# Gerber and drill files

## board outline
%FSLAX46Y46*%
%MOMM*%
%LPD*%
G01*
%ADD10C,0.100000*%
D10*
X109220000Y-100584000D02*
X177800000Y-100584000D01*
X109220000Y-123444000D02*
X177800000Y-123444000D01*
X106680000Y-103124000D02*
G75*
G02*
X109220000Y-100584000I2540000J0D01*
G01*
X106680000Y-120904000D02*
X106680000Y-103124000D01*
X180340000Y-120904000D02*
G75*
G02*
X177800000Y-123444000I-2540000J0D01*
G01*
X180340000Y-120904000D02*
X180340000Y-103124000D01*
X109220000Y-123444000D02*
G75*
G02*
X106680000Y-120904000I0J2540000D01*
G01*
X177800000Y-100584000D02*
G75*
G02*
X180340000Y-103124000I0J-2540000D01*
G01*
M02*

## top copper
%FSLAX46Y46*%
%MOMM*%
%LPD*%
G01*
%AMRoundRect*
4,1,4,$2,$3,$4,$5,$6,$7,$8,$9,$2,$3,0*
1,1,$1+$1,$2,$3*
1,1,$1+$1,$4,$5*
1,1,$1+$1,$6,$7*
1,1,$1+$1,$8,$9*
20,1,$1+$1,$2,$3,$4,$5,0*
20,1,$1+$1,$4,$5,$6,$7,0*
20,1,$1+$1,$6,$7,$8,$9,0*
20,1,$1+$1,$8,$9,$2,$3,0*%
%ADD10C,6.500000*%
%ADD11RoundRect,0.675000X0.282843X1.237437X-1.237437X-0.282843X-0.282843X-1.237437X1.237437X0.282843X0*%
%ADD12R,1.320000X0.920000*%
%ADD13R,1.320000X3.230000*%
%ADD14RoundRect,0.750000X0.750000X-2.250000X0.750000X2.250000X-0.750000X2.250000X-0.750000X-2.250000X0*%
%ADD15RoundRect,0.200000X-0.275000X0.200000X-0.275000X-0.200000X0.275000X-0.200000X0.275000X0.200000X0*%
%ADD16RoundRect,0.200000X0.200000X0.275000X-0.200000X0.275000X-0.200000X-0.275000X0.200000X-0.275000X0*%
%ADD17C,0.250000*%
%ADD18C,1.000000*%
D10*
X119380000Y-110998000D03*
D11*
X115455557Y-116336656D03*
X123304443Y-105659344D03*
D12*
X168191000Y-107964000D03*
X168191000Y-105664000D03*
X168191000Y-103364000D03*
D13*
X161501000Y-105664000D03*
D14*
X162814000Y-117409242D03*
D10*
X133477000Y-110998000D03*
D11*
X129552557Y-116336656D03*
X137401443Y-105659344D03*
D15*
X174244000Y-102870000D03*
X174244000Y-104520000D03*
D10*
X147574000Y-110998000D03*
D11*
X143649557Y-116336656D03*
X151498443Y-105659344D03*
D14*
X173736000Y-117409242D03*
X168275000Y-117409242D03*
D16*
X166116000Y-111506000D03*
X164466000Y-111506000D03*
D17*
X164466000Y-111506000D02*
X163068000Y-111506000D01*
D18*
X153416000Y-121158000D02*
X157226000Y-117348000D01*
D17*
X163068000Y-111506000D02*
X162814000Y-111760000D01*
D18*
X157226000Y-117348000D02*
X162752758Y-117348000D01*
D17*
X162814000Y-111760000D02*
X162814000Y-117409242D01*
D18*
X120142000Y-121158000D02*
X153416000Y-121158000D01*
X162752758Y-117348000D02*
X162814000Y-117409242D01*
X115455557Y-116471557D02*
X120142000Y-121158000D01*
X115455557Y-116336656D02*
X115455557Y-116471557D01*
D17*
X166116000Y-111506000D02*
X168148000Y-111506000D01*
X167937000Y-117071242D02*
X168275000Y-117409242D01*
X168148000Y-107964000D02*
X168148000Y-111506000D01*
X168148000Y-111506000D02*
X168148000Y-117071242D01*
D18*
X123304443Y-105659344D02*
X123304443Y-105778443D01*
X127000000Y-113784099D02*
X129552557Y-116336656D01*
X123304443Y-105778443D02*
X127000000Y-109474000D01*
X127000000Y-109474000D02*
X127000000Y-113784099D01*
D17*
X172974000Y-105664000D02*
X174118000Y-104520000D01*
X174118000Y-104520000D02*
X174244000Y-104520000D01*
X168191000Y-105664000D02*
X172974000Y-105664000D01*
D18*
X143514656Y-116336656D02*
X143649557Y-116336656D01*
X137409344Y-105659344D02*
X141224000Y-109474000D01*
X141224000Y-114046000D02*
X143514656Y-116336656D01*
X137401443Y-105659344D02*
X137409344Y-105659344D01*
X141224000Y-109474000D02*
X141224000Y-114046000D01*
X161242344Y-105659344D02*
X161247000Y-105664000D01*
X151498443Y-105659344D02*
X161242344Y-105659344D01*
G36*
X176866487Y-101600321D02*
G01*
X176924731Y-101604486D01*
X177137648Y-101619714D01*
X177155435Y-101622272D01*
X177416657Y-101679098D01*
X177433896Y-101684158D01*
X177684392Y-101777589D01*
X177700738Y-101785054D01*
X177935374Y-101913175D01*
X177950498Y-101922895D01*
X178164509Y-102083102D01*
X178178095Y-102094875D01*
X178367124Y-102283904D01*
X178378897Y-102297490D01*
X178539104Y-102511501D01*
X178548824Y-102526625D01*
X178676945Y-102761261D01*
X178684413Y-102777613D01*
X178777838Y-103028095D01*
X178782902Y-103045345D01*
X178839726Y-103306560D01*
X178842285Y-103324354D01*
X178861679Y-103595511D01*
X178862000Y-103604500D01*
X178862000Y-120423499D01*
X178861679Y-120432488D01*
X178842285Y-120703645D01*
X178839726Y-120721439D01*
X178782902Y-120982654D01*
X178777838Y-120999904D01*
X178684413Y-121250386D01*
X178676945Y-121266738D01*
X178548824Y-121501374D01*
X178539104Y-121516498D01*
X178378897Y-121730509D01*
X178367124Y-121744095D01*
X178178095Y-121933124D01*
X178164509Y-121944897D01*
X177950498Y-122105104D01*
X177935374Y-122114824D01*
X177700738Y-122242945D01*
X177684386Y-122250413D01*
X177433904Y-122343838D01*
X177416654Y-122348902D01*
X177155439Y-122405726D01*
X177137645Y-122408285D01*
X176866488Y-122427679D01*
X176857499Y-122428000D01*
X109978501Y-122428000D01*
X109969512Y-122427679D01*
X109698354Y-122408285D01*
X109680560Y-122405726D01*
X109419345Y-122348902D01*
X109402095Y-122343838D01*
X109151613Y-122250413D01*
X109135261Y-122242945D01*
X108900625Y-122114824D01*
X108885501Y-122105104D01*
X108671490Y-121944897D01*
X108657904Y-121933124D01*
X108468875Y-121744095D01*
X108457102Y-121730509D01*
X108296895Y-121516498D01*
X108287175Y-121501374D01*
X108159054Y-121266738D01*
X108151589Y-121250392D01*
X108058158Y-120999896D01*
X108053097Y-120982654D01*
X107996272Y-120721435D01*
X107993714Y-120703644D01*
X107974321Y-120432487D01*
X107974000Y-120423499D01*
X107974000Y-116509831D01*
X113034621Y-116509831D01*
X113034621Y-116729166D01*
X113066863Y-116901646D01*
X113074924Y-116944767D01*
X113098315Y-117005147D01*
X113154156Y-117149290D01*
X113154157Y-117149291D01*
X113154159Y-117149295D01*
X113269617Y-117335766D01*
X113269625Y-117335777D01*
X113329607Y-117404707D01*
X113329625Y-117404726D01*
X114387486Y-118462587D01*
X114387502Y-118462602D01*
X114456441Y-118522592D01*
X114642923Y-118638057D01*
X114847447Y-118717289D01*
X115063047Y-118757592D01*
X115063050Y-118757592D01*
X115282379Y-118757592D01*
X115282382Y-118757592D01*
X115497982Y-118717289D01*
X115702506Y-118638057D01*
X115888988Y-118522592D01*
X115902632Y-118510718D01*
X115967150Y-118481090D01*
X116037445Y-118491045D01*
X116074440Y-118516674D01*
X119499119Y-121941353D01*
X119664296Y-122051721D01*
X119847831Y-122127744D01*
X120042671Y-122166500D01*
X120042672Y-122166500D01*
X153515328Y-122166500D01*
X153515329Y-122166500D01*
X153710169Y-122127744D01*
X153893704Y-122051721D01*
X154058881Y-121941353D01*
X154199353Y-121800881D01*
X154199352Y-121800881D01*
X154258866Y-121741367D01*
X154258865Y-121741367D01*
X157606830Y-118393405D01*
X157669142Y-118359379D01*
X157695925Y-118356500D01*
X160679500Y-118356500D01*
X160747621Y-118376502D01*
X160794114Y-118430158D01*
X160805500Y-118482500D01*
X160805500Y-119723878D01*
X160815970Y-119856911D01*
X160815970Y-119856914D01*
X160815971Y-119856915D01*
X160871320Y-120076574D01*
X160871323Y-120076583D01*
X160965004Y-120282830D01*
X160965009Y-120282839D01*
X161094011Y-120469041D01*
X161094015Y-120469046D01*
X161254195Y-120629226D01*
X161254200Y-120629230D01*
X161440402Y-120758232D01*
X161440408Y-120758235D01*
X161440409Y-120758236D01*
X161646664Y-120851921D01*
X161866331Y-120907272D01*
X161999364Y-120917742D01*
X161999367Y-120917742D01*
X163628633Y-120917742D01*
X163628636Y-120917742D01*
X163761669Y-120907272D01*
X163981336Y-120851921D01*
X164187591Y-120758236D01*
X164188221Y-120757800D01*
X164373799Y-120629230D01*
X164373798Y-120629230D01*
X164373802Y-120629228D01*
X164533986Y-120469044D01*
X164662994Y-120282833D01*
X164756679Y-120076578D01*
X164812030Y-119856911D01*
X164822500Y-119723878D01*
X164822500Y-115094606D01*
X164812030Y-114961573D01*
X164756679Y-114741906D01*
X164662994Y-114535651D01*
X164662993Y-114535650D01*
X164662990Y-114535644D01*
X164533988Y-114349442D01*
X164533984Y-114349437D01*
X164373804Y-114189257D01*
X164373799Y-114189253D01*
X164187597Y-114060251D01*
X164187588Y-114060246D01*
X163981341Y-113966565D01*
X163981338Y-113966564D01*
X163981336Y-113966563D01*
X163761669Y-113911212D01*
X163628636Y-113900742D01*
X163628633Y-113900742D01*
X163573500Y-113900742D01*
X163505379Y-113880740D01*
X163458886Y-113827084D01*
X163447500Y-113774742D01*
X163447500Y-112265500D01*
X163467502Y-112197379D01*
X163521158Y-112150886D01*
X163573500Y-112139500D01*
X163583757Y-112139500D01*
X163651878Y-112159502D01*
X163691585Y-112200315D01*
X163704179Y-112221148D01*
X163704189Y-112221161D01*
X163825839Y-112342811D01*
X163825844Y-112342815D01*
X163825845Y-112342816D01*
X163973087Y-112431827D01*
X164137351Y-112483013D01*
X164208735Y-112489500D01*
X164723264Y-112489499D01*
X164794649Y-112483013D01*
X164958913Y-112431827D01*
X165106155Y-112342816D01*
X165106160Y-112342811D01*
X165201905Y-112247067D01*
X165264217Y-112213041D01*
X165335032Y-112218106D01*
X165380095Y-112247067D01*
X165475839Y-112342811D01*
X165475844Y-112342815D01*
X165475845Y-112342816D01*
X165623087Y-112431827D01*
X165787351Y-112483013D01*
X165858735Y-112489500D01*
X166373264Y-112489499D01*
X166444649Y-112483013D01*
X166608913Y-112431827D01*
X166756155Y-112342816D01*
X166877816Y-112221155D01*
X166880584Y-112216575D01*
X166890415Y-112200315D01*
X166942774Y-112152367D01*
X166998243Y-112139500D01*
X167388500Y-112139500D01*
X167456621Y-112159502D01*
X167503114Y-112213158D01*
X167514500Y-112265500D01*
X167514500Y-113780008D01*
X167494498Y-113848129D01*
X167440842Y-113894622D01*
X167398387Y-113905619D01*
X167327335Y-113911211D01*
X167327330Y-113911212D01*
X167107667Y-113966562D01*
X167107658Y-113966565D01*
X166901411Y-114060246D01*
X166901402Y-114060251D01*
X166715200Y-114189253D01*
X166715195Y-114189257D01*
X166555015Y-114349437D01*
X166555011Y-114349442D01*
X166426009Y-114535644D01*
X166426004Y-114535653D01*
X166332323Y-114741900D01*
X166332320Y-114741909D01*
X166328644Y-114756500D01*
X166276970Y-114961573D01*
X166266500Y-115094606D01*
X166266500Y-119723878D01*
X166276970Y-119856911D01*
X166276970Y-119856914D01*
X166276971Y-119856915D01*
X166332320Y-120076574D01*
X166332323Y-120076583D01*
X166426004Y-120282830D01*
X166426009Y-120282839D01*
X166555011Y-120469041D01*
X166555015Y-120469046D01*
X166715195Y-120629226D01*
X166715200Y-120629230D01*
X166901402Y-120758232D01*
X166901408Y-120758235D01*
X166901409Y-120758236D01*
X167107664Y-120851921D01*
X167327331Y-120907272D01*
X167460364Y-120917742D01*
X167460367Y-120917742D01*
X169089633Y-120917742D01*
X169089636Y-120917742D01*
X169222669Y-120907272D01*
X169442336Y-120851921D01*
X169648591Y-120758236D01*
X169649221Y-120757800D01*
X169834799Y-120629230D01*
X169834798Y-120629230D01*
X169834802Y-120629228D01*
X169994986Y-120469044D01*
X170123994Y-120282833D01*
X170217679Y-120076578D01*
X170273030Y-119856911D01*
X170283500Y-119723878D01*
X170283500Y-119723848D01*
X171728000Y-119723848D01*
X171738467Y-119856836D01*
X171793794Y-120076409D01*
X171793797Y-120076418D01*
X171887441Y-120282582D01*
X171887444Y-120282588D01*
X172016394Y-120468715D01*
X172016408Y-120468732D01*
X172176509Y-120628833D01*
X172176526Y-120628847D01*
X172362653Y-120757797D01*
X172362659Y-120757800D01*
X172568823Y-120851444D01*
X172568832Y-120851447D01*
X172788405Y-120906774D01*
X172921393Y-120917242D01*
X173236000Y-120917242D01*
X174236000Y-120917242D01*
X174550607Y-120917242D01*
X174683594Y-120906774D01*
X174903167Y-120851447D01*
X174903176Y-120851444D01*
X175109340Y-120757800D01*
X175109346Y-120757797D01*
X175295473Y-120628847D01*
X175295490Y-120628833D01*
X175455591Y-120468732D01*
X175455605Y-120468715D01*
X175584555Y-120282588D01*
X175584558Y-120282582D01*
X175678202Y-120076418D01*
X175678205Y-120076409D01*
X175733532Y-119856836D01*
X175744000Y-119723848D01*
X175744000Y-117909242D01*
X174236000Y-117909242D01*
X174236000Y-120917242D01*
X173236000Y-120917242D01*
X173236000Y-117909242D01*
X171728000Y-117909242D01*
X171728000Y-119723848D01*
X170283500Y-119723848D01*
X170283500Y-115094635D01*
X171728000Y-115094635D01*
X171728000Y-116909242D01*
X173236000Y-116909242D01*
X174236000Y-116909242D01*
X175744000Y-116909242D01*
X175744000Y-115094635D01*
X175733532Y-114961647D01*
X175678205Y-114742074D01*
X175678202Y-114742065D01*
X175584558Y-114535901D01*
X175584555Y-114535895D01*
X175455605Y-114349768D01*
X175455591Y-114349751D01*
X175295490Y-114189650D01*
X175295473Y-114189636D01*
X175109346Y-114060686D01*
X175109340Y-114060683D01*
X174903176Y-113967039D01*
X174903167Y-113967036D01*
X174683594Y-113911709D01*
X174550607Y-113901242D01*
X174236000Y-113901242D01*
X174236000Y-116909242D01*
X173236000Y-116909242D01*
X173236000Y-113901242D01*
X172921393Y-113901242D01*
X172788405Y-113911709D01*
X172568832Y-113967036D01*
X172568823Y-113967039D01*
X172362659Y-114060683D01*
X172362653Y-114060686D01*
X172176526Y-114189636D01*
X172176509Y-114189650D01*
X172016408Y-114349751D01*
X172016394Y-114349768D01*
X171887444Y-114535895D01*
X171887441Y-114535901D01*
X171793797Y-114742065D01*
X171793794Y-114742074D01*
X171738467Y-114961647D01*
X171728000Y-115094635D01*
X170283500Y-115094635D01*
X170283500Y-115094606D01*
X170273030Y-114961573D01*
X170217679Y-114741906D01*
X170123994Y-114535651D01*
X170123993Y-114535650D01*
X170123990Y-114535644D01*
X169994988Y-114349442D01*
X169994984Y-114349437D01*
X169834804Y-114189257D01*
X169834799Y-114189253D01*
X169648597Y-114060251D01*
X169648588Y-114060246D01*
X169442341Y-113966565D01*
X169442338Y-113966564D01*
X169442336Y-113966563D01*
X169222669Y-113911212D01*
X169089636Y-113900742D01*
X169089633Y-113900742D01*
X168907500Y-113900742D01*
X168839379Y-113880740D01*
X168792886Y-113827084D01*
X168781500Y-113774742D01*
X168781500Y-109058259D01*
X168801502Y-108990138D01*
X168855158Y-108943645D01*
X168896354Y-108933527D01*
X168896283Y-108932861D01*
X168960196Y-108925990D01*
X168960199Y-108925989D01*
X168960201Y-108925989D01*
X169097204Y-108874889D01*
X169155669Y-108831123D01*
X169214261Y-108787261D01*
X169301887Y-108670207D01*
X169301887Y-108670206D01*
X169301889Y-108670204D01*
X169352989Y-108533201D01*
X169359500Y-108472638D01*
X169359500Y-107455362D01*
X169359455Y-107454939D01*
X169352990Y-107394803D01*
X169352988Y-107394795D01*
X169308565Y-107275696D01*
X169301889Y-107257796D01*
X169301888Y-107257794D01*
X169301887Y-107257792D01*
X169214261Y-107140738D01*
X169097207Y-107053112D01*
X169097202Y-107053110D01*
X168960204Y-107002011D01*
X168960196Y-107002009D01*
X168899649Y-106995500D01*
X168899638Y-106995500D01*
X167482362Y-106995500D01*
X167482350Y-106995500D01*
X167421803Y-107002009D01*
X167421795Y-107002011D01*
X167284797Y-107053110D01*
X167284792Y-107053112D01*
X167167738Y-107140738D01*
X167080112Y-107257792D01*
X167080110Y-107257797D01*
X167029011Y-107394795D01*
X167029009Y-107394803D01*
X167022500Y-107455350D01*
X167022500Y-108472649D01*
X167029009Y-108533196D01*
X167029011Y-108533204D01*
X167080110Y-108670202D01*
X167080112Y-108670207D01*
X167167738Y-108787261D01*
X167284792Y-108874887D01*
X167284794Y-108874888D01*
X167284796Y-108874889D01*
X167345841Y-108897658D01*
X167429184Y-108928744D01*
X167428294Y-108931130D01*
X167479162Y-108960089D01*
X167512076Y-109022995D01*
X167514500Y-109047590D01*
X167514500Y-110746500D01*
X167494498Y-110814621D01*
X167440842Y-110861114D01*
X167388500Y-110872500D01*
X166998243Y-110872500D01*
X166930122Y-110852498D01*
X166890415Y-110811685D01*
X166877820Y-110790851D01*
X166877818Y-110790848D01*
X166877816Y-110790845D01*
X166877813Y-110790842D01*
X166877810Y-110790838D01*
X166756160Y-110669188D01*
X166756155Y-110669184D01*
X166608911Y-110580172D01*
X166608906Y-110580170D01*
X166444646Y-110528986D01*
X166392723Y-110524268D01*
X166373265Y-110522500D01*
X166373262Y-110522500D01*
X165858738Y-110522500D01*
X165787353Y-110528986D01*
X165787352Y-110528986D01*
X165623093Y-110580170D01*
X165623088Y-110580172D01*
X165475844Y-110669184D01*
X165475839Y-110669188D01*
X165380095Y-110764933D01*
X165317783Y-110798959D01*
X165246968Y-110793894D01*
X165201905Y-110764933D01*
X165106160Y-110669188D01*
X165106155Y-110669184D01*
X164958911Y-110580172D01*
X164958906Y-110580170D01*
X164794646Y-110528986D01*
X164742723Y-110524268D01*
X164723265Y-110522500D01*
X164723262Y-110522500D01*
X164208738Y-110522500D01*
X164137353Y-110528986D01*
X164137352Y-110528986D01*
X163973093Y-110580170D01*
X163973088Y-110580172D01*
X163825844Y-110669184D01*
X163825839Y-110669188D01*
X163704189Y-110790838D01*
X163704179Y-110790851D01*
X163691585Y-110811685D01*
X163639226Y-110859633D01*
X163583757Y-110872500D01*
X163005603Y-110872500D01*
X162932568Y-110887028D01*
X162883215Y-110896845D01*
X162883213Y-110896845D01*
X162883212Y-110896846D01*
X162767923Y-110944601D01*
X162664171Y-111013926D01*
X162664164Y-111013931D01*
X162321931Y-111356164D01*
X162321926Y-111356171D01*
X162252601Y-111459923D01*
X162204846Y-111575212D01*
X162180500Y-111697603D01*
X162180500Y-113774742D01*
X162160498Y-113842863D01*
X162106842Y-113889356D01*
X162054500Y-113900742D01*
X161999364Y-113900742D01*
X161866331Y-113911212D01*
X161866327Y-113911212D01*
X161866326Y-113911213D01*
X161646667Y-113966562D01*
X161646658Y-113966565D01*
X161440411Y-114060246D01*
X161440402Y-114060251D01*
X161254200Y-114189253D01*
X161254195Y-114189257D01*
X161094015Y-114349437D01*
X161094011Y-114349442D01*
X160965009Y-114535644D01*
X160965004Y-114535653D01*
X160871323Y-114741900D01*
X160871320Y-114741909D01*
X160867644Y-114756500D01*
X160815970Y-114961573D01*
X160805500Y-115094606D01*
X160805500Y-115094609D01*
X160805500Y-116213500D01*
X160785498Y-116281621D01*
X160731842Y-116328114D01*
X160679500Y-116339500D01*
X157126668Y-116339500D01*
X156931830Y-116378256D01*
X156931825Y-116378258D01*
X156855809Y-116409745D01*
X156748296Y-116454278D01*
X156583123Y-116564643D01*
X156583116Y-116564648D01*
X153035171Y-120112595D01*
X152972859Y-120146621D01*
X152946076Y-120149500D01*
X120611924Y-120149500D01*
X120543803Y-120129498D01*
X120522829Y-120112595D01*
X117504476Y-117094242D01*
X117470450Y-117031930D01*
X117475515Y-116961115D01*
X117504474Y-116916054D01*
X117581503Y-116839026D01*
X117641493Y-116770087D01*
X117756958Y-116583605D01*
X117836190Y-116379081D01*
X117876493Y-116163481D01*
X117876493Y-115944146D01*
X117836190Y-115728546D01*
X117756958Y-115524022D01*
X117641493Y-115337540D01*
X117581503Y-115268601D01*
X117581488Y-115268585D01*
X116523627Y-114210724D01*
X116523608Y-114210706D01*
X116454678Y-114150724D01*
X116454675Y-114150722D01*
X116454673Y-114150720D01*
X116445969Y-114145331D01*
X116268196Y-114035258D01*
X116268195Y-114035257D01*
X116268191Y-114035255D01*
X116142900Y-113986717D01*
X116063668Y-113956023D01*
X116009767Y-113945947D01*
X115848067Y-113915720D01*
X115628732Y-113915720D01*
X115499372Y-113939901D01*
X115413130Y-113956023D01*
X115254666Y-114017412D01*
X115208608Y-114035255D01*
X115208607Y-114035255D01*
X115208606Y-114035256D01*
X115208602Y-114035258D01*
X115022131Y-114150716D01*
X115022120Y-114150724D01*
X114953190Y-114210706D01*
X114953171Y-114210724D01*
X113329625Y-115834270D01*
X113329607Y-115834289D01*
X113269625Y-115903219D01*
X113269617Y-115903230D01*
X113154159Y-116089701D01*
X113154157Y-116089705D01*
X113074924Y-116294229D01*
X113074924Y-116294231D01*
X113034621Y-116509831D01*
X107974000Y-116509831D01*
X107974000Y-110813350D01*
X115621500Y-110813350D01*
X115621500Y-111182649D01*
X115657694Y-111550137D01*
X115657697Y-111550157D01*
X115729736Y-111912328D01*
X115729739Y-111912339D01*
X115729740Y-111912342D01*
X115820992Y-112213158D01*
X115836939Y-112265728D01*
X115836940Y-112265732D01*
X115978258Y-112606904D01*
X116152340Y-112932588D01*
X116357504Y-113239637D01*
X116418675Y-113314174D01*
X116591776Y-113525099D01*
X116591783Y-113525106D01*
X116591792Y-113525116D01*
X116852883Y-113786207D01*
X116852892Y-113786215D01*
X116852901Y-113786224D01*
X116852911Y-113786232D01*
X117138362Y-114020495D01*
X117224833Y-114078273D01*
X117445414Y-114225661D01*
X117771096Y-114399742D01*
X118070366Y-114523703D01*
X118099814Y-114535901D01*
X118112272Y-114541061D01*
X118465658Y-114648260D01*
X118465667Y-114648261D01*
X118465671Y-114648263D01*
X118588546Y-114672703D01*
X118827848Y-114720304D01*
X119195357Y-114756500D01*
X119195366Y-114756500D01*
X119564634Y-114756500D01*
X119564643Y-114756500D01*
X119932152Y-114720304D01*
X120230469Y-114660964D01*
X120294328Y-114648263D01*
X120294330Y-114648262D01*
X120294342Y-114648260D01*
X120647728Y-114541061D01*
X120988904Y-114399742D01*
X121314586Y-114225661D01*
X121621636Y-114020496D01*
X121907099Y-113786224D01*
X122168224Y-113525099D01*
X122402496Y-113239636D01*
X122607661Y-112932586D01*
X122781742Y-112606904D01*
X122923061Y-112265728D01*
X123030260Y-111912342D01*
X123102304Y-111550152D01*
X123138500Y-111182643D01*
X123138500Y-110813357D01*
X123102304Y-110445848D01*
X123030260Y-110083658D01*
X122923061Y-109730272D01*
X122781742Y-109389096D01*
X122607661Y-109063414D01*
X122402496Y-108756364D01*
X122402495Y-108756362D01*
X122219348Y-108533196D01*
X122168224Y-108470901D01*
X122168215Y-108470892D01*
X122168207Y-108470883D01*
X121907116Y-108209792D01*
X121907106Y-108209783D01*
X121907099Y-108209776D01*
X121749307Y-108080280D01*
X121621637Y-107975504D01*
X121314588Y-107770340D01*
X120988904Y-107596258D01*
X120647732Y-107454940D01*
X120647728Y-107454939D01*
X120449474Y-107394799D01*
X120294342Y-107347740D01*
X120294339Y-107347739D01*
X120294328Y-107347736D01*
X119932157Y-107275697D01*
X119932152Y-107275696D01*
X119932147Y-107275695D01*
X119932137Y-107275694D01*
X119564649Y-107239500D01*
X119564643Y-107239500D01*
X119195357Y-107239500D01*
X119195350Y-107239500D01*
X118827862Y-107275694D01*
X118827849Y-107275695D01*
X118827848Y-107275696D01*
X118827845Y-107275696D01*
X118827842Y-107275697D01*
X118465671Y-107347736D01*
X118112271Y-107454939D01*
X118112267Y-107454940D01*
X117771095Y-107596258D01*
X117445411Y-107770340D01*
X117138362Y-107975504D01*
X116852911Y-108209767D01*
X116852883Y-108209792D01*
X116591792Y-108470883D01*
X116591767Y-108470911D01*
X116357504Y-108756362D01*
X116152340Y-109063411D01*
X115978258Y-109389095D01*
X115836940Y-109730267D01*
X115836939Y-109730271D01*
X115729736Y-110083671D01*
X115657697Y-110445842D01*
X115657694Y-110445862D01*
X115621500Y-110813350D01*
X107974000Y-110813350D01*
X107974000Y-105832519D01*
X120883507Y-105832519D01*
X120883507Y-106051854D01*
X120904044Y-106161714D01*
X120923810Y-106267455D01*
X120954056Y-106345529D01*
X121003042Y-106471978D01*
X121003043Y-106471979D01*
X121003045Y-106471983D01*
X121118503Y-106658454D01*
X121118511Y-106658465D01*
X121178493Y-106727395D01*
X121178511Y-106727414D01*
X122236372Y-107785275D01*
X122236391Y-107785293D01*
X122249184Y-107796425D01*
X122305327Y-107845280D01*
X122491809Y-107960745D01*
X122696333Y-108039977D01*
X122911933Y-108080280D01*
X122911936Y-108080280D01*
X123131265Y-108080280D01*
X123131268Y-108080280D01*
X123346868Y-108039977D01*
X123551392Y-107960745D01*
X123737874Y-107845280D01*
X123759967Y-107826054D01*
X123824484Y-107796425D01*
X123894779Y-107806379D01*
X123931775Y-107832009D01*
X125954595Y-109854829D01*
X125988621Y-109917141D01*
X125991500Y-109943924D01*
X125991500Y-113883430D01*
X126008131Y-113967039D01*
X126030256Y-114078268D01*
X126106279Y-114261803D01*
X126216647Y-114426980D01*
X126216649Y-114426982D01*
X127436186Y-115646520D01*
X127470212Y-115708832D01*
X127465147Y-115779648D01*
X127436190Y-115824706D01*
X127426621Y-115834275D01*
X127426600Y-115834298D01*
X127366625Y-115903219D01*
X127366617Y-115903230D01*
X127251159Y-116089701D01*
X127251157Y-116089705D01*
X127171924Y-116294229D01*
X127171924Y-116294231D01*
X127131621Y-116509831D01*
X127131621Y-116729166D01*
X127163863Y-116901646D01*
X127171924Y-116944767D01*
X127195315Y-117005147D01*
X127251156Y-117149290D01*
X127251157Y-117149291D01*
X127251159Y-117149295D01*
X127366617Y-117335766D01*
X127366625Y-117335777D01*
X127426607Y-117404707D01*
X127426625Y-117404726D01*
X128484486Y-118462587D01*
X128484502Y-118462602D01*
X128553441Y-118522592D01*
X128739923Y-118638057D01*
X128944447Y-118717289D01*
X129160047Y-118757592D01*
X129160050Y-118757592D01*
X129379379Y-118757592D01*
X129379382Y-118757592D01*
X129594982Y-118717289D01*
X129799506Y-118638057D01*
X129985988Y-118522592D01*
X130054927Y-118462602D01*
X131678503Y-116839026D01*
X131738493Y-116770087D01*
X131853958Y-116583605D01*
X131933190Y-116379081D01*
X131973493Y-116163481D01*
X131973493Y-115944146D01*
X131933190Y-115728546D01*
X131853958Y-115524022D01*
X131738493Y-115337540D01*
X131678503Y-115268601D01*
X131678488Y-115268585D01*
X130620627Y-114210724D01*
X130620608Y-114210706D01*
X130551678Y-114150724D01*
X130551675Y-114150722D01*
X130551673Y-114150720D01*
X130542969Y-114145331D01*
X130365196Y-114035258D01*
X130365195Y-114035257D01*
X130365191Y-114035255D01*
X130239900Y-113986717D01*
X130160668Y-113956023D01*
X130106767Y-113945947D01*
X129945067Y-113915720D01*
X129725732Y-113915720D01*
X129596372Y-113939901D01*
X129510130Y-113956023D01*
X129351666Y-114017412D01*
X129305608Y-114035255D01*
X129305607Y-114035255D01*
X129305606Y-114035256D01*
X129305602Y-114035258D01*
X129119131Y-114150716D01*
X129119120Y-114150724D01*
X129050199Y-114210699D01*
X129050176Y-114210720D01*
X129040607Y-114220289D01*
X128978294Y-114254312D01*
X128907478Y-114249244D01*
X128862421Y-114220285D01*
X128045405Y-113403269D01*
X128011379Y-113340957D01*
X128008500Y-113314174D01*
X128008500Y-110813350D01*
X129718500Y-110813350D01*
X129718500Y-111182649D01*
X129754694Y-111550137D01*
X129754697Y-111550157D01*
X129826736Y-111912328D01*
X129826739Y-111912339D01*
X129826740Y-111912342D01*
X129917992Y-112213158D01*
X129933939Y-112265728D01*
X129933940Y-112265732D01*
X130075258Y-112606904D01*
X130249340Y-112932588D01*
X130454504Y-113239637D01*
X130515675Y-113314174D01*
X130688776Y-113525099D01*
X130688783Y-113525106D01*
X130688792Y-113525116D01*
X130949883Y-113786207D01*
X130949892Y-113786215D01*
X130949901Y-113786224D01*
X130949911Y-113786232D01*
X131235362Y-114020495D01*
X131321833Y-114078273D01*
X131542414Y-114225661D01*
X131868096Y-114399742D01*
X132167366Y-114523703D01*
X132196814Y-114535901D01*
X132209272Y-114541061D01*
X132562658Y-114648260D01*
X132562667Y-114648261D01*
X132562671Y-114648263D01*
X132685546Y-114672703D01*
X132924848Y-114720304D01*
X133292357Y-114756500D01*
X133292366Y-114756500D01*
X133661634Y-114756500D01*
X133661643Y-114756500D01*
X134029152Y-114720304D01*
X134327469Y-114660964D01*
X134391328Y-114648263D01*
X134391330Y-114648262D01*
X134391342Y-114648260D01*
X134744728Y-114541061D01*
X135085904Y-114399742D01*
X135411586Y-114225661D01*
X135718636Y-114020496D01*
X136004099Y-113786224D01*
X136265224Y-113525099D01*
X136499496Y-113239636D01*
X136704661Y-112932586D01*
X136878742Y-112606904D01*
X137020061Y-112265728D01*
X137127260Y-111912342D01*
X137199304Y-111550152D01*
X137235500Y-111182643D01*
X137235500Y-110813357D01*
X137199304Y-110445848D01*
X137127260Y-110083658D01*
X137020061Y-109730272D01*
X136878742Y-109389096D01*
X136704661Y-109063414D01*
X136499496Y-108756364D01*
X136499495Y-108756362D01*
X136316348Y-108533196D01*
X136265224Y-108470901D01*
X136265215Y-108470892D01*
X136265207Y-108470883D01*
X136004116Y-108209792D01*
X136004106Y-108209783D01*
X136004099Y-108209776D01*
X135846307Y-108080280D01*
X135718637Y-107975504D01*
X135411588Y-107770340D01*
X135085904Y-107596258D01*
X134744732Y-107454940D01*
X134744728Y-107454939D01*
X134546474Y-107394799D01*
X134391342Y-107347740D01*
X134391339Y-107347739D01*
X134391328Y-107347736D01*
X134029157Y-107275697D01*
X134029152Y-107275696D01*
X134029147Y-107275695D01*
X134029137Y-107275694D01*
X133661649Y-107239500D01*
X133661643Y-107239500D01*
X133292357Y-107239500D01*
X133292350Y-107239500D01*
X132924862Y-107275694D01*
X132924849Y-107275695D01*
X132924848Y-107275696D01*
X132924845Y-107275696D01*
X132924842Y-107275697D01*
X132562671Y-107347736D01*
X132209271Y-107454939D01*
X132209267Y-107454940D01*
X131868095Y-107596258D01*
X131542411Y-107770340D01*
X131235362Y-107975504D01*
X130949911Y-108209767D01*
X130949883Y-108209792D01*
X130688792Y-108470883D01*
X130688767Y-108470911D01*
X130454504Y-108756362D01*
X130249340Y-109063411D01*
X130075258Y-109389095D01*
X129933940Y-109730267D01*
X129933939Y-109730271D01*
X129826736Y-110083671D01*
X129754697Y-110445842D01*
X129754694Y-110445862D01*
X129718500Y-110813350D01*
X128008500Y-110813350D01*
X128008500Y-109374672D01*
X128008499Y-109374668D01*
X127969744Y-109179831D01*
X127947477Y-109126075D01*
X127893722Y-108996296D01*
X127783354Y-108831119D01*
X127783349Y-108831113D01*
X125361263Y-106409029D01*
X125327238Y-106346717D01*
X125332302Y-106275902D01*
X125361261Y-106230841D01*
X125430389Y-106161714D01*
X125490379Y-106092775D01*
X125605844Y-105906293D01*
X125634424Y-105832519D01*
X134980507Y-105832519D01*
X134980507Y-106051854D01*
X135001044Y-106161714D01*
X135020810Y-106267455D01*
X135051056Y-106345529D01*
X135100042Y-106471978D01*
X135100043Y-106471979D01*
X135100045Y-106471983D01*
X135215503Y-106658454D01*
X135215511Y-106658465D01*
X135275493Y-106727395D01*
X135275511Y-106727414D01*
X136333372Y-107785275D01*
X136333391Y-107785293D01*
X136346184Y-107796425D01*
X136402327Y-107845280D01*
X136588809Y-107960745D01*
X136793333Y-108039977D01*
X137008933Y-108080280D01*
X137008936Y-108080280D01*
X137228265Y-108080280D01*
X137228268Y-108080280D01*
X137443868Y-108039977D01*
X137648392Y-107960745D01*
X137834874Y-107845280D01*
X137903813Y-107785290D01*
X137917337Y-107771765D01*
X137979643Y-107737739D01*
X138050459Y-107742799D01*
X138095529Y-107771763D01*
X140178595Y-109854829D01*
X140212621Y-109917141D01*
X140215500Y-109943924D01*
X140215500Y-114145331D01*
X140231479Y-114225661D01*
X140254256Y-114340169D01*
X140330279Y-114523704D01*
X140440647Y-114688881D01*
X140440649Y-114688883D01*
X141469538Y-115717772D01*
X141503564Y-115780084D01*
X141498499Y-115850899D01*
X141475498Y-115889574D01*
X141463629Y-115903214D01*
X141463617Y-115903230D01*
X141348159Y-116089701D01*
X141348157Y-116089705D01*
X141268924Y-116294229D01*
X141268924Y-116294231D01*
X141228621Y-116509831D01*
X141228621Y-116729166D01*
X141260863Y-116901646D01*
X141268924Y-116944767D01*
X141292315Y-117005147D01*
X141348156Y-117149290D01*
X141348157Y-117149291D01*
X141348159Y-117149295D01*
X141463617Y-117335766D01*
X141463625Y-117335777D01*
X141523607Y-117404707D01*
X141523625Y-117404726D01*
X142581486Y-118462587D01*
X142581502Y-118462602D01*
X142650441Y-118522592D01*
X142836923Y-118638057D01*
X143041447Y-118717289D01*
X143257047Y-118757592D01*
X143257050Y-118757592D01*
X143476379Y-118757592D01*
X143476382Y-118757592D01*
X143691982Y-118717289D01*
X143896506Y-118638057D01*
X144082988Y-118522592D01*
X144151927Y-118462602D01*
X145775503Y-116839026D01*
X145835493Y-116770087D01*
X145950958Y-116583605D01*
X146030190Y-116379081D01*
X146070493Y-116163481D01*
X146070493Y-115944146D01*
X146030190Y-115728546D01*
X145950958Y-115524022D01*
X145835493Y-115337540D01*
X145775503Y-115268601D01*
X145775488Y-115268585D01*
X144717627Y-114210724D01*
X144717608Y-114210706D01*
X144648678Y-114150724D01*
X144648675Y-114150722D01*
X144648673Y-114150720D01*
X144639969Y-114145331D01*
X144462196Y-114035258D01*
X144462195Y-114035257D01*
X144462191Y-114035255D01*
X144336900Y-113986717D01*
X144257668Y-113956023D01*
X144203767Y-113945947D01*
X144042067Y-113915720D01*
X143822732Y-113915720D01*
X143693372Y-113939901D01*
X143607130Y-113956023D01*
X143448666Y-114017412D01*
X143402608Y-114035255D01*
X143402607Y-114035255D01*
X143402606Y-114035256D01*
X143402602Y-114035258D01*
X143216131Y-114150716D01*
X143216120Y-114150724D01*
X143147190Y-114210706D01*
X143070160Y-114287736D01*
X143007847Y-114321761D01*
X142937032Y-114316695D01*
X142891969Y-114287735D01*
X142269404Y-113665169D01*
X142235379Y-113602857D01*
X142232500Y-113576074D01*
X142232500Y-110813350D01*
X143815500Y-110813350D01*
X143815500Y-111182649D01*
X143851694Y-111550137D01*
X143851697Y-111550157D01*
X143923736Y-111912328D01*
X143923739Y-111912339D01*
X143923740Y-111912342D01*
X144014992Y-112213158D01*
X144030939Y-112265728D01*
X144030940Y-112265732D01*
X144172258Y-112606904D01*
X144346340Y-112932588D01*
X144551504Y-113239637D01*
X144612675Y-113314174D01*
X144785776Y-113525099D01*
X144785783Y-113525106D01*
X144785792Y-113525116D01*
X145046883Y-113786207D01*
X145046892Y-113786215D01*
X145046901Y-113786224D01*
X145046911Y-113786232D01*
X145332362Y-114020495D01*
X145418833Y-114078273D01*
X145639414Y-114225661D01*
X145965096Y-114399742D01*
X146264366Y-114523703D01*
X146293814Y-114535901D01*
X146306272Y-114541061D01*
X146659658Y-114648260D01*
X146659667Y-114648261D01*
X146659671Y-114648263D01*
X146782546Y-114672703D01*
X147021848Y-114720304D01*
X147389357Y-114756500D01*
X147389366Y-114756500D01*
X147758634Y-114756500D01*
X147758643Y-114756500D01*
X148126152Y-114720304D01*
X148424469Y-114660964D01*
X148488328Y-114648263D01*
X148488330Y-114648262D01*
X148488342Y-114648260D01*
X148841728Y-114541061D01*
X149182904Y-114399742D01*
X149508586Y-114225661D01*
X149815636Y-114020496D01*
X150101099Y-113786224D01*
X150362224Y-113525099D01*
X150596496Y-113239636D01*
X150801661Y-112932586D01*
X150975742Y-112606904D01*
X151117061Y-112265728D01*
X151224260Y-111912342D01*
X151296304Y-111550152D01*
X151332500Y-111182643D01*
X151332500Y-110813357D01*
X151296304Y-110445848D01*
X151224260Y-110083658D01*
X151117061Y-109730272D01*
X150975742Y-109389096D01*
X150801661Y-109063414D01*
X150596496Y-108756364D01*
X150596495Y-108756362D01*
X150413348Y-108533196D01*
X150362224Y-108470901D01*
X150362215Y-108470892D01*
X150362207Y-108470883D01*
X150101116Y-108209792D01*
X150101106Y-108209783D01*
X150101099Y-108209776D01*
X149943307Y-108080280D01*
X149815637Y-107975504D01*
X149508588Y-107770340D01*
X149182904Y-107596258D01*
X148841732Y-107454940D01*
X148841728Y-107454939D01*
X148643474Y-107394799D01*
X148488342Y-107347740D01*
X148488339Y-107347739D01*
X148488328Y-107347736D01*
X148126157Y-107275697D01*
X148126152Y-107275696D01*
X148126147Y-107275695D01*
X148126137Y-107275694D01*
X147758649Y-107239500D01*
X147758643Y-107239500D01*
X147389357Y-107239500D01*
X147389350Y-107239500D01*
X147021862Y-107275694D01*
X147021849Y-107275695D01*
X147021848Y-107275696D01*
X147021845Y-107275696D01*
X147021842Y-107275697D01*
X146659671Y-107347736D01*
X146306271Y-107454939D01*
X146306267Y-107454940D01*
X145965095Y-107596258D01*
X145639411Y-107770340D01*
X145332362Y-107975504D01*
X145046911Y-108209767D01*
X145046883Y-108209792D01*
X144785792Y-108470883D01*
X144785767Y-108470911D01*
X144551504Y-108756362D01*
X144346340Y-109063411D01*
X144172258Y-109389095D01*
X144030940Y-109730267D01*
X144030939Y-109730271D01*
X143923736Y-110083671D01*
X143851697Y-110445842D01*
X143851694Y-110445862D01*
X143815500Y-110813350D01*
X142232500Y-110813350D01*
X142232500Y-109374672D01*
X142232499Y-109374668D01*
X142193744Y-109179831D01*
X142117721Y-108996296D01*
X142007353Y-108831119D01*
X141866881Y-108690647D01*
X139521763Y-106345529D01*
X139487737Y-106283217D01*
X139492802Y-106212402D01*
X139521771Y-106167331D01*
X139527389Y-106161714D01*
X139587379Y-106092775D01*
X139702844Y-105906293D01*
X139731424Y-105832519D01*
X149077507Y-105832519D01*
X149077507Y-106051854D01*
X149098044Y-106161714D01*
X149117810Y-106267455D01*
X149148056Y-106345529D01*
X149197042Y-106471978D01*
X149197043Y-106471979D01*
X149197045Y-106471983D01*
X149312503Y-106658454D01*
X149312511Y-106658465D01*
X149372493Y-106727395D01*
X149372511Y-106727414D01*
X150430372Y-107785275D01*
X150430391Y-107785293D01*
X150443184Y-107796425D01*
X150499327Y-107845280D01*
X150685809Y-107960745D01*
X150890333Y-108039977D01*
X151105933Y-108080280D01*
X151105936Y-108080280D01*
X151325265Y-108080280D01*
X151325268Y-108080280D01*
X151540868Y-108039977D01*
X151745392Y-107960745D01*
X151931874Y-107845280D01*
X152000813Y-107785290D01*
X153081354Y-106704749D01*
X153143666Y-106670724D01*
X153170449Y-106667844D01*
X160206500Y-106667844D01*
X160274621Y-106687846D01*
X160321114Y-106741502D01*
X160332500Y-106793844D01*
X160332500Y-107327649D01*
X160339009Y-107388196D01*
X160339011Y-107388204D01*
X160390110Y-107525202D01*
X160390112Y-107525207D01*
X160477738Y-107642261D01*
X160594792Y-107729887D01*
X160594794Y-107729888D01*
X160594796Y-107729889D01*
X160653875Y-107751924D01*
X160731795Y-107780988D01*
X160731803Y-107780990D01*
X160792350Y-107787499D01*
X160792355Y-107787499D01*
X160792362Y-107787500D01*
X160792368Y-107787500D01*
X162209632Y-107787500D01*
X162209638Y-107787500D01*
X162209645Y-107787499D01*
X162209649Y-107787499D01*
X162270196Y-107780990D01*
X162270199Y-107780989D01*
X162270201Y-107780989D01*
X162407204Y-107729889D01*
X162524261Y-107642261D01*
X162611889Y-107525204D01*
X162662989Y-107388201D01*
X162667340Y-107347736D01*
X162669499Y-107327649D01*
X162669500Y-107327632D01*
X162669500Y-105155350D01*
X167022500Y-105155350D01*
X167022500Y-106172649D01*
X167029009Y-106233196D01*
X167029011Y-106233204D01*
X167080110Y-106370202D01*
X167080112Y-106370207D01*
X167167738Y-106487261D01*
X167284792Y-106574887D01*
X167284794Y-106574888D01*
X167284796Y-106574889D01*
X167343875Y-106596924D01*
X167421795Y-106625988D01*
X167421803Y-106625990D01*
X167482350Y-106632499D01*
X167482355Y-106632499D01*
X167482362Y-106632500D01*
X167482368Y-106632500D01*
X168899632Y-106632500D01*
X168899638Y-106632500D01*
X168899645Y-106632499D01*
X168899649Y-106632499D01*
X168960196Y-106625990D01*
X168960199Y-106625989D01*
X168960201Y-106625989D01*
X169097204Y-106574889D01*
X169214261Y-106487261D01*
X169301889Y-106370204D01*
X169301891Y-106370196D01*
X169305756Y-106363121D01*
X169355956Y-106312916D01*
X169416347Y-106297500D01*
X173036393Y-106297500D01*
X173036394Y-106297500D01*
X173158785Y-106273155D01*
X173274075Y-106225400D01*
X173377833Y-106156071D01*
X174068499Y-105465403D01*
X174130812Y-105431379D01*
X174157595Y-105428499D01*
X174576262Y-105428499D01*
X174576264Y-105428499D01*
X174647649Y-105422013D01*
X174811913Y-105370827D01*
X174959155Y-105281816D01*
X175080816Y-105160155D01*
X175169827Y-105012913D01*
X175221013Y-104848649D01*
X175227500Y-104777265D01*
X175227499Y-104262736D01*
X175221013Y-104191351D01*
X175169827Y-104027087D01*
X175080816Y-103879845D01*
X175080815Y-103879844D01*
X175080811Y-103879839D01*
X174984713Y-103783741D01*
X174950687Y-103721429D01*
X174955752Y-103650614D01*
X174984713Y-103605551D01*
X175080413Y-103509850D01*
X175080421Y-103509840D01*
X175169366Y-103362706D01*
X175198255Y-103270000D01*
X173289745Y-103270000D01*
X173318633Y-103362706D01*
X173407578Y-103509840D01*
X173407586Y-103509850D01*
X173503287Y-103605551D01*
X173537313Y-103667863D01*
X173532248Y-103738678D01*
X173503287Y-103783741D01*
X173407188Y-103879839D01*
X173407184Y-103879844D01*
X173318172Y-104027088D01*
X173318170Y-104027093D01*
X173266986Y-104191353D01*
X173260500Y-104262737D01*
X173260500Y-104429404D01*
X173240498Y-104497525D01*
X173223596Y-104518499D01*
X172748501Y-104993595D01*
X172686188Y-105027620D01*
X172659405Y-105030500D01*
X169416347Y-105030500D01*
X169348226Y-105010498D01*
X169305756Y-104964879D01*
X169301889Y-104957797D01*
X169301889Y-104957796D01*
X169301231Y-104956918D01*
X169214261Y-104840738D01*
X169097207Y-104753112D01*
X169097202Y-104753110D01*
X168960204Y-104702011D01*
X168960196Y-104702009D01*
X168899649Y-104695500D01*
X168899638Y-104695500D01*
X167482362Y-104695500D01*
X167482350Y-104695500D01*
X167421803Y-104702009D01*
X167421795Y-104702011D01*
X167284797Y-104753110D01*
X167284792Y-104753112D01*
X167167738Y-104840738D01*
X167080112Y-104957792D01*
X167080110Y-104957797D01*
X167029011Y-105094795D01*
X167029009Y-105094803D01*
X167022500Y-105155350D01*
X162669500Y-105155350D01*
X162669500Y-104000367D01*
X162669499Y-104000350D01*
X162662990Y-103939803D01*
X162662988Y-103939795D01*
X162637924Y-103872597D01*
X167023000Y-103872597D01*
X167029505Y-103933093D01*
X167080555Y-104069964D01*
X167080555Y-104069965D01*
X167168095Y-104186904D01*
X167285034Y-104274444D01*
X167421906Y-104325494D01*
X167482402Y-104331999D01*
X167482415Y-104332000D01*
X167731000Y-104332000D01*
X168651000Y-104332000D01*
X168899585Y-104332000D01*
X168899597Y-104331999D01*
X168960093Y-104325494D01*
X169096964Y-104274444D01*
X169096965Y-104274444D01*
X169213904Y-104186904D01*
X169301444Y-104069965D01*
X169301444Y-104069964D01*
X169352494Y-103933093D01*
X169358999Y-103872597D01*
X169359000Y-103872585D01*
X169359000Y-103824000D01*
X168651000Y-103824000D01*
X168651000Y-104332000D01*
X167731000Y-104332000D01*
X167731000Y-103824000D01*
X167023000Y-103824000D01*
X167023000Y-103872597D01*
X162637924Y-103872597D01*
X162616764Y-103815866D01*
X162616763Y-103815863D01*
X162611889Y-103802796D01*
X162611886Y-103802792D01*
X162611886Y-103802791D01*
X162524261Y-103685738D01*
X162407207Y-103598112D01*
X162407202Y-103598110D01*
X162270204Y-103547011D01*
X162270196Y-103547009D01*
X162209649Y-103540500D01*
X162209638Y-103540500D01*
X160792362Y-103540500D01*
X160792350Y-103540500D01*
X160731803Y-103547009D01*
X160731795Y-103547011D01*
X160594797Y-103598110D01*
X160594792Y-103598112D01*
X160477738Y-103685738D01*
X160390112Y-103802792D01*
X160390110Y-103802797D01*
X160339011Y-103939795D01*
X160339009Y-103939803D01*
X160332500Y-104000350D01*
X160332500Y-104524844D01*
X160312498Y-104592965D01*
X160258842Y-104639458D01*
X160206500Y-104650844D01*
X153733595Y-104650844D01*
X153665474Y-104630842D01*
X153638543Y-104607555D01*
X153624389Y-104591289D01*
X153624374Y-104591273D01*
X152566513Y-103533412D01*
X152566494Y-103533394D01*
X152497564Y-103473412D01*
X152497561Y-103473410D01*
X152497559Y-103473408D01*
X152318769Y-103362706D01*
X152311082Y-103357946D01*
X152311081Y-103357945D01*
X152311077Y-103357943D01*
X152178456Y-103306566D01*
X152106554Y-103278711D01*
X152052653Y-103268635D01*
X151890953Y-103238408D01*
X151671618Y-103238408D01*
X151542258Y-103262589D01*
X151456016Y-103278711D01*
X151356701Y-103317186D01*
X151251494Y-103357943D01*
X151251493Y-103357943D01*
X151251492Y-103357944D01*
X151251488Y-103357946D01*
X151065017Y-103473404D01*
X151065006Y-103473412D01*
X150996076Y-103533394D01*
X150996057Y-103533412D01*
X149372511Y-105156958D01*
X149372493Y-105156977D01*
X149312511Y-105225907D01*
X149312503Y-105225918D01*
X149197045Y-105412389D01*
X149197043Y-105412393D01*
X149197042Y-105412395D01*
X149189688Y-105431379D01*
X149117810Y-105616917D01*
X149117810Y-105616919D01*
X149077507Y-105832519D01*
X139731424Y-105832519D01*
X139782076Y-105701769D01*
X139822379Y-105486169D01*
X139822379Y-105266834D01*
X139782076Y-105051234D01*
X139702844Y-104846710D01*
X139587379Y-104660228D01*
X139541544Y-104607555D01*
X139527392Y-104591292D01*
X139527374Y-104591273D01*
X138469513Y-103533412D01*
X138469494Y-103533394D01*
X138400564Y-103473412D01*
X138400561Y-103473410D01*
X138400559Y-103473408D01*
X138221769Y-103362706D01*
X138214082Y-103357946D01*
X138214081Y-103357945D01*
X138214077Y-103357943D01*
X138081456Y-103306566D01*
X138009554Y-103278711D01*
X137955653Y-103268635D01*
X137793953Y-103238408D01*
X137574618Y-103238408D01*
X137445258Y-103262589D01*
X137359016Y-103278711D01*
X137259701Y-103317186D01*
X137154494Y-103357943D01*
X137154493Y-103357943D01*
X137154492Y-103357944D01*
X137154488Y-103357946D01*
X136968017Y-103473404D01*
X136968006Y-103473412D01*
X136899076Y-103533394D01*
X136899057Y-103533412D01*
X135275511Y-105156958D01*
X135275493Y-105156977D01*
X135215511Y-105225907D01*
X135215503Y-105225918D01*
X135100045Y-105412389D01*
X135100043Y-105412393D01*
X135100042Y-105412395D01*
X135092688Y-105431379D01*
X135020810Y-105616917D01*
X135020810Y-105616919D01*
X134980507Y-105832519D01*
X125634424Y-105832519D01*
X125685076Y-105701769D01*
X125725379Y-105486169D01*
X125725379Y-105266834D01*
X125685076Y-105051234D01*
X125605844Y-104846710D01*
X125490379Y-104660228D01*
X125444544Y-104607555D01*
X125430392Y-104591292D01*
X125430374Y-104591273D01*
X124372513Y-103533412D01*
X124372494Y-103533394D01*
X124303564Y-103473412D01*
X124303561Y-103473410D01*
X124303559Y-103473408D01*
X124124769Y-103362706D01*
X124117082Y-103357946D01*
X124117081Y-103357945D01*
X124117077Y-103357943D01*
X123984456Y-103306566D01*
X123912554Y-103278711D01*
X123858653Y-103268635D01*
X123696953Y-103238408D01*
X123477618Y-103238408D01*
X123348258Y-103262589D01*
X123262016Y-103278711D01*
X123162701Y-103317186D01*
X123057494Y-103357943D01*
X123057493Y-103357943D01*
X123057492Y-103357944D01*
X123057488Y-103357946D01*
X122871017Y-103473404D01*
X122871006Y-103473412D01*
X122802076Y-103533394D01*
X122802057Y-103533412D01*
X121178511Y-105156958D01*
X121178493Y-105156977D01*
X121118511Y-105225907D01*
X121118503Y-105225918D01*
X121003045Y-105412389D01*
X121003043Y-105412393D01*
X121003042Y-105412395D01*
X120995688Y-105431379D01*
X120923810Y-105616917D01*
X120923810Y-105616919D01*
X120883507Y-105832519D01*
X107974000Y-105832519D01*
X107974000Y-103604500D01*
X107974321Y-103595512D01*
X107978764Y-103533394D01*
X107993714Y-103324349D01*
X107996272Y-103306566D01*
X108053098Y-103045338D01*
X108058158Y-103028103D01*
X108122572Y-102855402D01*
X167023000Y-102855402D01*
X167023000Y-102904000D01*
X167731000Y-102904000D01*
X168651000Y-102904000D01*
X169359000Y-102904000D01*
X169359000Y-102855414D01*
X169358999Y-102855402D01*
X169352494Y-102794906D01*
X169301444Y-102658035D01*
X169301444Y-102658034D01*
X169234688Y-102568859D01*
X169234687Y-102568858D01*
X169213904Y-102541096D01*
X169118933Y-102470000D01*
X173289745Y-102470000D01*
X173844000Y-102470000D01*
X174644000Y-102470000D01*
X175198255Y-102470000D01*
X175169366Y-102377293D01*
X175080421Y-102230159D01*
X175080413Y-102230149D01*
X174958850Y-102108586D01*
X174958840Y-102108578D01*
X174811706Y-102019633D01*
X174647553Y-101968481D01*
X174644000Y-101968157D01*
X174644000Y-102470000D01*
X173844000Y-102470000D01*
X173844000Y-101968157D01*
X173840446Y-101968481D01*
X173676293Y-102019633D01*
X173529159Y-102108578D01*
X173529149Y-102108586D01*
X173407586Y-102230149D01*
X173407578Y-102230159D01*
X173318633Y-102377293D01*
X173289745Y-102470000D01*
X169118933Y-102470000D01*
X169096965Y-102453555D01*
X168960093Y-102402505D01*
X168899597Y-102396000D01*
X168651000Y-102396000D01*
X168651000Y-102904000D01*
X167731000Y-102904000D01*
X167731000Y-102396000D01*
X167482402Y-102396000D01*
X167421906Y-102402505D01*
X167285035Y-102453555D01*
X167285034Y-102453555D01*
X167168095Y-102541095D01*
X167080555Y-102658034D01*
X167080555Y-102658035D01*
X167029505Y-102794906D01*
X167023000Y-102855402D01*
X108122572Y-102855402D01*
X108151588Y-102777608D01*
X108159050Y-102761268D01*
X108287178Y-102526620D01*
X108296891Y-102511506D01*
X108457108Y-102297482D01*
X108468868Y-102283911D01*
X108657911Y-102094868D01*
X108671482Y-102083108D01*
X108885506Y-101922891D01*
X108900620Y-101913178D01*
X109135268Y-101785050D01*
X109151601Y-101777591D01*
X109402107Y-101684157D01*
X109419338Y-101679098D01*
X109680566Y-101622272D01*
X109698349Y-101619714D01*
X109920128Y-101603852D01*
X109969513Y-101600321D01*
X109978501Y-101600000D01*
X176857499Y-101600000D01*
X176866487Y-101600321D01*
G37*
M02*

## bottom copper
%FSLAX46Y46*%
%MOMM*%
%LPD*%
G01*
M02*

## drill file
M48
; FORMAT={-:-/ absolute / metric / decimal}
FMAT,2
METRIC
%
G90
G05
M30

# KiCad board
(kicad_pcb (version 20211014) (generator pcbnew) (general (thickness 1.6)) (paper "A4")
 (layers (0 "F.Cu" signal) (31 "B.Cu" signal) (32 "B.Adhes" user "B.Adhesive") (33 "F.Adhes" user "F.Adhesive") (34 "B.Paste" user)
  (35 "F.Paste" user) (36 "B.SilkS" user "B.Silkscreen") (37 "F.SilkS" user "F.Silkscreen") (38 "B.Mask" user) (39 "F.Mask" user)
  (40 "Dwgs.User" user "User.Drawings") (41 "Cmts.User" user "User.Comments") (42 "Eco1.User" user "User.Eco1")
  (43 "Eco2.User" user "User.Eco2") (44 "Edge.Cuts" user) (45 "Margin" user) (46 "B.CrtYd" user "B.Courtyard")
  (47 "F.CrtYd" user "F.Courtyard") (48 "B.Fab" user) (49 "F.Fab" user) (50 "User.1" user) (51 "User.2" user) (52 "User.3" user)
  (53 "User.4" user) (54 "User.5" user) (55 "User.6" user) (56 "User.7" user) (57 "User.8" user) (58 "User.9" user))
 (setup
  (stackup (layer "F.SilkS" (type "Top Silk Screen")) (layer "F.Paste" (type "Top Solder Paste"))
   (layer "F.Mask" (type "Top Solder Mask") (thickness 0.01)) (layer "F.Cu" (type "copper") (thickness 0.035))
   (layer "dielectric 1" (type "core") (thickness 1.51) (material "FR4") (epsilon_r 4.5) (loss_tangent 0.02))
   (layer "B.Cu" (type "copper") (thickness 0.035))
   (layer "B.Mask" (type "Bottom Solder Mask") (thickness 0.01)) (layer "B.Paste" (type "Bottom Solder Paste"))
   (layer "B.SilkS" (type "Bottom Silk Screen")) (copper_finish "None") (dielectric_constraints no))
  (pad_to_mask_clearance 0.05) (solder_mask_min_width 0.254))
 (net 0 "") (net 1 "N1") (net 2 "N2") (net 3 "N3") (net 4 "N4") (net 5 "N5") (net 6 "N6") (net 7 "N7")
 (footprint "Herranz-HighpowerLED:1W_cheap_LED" (layer "F.Cu") (at 119.38 110.998 -135)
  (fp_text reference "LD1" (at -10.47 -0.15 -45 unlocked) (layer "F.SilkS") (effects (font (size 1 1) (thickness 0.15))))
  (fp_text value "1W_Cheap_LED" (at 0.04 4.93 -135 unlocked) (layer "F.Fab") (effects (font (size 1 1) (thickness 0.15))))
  (pad "" smd circle (at 0 0 225) (size 6.5 6.5) (layers "F.Cu" "F.Paste" "F.Mask"))
  (pad "1" smd roundrect (at 6.55 -1 225) (size 3.5 2.7) (layers "F.Cu" "F.Paste" "F.Mask") (roundrect_rratio 0.25) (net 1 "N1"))
  (pad "2" smd roundrect (at -6.55 1 225) (size 3.5 2.7) (layers "F.Cu" "F.Paste" "F.Mask") (roundrect_rratio 0.25) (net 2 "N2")))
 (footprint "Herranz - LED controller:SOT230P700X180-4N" (layer "F.Cu") (at 164.846 105.664 180)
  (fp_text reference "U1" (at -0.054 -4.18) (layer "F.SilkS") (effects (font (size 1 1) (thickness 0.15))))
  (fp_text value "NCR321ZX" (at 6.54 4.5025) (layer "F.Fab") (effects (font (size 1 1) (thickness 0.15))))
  (pad "1" smd rect (at -3.345 -2.3 180) (size 1.32 0.92) (layers "F.Cu" "F.Paste" "F.Mask") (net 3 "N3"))
  (pad "2" smd rect (at -3.345 0 180) (size 1.32 0.92) (layers "F.Cu" "F.Paste" "F.Mask") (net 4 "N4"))
  (pad "3" smd rect (at -3.345 2.3 180) (size 1.32 0.92) (layers "F.Cu" "F.Paste" "F.Mask") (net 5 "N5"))
  (pad "4" smd rect (at 3.345 0 180) (size 1.32 3.23) (layers "F.Cu" "F.Paste" "F.Mask") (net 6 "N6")))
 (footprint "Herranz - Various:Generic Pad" (layer "F.Cu") (at 162.814 117.409242 90)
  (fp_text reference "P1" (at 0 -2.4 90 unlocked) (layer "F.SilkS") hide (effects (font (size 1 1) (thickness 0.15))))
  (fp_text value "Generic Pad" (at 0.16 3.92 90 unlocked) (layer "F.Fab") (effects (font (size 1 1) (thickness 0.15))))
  (pad "1" smd roundrect (at 0 0 90) (size 6 3) (layers "F.Cu" "F.Paste" "F.Mask") (roundrect_rratio 0.25) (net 1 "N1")))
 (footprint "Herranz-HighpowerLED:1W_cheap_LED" (layer "F.Cu") (at 133.477 110.998 -135)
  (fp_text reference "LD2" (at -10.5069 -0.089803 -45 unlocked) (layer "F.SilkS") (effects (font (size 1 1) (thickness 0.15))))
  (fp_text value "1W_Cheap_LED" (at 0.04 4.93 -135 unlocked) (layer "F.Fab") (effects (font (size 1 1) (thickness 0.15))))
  (pad "" smd circle (at 0 0 225) (size 6.5 6.5) (layers "F.Cu" "F.Paste" "F.Mask"))
  (pad "1" smd roundrect (at 6.55 -1 225) (size 3.5 2.7) (layers "F.Cu" "F.Paste" "F.Mask") (roundrect_rratio 0.25) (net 2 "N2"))
  (pad "2" smd roundrect (at -6.55 1 225) (size 3.5 2.7) (layers "F.Cu" "F.Paste" "F.Mask") (roundrect_rratio 0.25) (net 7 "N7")))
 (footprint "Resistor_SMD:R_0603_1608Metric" (layer "F.Cu") (at 174.244 103.695 -90)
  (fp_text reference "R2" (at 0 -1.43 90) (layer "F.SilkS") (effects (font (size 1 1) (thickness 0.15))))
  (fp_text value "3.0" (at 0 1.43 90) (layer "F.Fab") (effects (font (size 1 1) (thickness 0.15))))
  (pad "1" smd roundrect locked (at -0.825 0 270) (size 0.8 0.95) (layers "F.Cu" "F.Paste" "F.Mask") (roundrect_rratio 0.25) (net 5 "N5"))
  (pad "2" smd roundrect locked (at 0.825 0 270) (size 0.8 0.95) (layers "F.Cu" "F.Paste" "F.Mask") (roundrect_rratio 0.25) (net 4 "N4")))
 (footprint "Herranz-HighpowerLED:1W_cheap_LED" (layer "F.Cu") (at 147.574 110.998 -135)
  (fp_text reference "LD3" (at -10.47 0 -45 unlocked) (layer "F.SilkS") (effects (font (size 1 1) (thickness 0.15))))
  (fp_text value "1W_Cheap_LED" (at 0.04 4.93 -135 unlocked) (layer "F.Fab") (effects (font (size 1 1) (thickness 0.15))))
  (pad "" smd circle (at 0 0 225) (size 6.5 6.5) (layers "F.Cu" "F.Paste" "F.Mask"))
  (pad "1" smd roundrect (at 6.55 -1 225) (size 3.5 2.7) (layers "F.Cu" "F.Paste" "F.Mask") (roundrect_rratio 0.25) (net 7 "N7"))
  (pad "2" smd roundrect (at -6.55 1 225) (size 3.5 2.7) (layers "F.Cu" "F.Paste" "F.Mask") (roundrect_rratio 0.25) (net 6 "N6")))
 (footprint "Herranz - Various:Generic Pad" (layer "F.Cu") (at 173.736 117.409242 90)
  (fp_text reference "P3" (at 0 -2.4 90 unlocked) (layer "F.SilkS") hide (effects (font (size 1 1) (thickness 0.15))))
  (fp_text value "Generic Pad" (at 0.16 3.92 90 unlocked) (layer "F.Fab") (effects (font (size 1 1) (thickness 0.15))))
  (pad "1" smd roundrect (at 0 0 90) (size 6 3) (layers "F.Cu" "F.Paste" "F.Mask") (roundrect_rratio 0.25) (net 5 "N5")))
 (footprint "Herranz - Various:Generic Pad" (layer "F.Cu") (at 168.275 117.409242 90)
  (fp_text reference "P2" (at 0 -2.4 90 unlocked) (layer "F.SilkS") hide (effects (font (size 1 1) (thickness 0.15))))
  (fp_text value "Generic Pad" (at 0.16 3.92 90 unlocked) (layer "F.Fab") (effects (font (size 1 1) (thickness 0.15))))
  (pad "1" smd roundrect (at 0 0 90) (size 6 3) (layers "F.Cu" "F.Paste" "F.Mask") (roundrect_rratio 0.25) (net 3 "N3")))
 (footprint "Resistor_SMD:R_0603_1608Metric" (layer "F.Cu") (at 165.291 111.506 180)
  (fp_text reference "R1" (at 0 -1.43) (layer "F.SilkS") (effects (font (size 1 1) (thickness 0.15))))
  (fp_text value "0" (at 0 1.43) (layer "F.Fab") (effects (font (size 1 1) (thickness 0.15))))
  (pad "1" smd roundrect locked (at -0.825 0 180) (size 0.8 0.95) (layers "F.Cu" "F.Paste" "F.Mask") (roundrect_rratio 0.25) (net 3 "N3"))
  (pad "2" smd roundrect locked (at 0.825 0 180) (size 0.8 0.95) (layers "F.Cu" "F.Paste" "F.Mask") (roundrect_rratio 0.25) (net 1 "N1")))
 (gr_line (start 109.22 100.584) (end 177.8 100.584) (layer "Edge.Cuts") (width 0.1))
 (gr_line (start 109.22 123.444) (end 177.8 123.444) (layer "Edge.Cuts") (width 0.1))
 (gr_arc (start 106.68 103.124) (mid 107.423949 101.327949) (end 109.22 100.584) (layer "Edge.Cuts") (width 0.1))
 (gr_line (start 106.68 120.904) (end 106.68 103.124) (layer "Edge.Cuts") (width 0.1))
 (gr_arc (start 180.34 120.904) (mid 179.596051 122.700051) (end 177.8 123.444) (layer "Edge.Cuts") (width 0.1))
 (gr_line (start 180.34 120.904) (end 180.34 103.124) (layer "Edge.Cuts") (width 0.1))
 (gr_arc (start 109.22 123.444) (mid 107.423949 122.700051) (end 106.68 120.904) (layer "Edge.Cuts") (width 0.1))
 (gr_arc (start 177.8 100.584) (mid 179.596051 101.327949) (end 180.34 103.124) (layer "Edge.Cuts") (width 0.1))
 (segment (start 164.466 111.506) (end 163.068 111.506) (width 0.25) (layer "F.Cu") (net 1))
 (segment (start 153.416 121.158) (end 157.226 117.348) (width 1) (layer "F.Cu") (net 1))
 (segment (start 163.068 111.506) (end 162.814 111.76) (width 0.25) (layer "F.Cu") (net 1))
 (segment (start 157.226 117.348) (end 162.752758 117.348) (width 1) (layer "F.Cu") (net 1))
 (segment (start 162.814 111.76) (end 162.814 117.409242) (width 0.25) (layer "F.Cu") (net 1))
 (segment (start 120.142 121.158) (end 153.416 121.158) (width 1) (layer "F.Cu") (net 1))
 (segment (start 162.752758 117.348) (end 162.814 117.409242) (width 1) (layer "F.Cu") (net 1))
 (segment (start 115.455557 116.471557) (end 120.142 121.158) (width 1) (layer "F.Cu") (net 1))
 (segment (start 115.455557 116.336656) (end 115.455557 116.471557) (width 1) (layer "F.Cu") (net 1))
 (segment (start 166.116 111.506) (end 168.148 111.506) (width 0.25) (layer "F.Cu") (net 3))
 (segment (start 167.937 117.071242) (end 168.275 117.409242) (width 0.25) (layer "F.Cu") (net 3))
 (segment (start 168.148 107.964) (end 168.148 111.506) (width 0.25) (layer "F.Cu") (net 3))
 (segment (start 168.148 111.506) (end 168.148 117.071242) (width 0.25) (layer "F.Cu") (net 3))
 (segment (start 123.304443 105.659344) (end 123.304443 105.778443) (width 1) (layer "F.Cu") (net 2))
 (segment (start 127 113.784099) (end 129.552557 116.336656) (width 1) (layer "F.Cu") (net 2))
 (segment (start 123.304443 105.778443) (end 127 109.474) (width 1) (layer "F.Cu") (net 2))
 (segment (start 127 109.474) (end 127 113.784099) (width 1) (layer "F.Cu") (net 2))
 (segment (start 172.974 105.664) (end 174.118 104.52) (width 0.25) (layer "F.Cu") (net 4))
 (segment (start 174.118 104.52) (end 174.244 104.52) (width 0.25) (layer "F.Cu") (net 4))
 (segment (start 168.191 105.664) (end 172.974 105.664) (width 0.25) (layer "F.Cu") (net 4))
 (segment (start 143.514656 116.336656) (end 143.649557 116.336656) (width 1) (layer "F.Cu") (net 7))
 (segment (start 137.409344 105.659344) (end 141.224 109.474) (width 1) (layer "F.Cu") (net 7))
 (segment (start 141.224 114.046) (end 143.514656 116.336656) (width 1) (layer "F.Cu") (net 7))
 (segment (start 137.401443 105.659344) (end 137.409344 105.659344) (width 1) (layer "F.Cu") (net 7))
 (segment (start 141.224 109.474) (end 141.224 114.046) (width 1) (layer "F.Cu") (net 7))
 (segment (start 161.242344 105.659344) (end 161.247 105.664) (width 1) (layer "F.Cu") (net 6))
 (segment (start 151.498443 105.659344) (end 161.242344 105.659344) (width 1) (layer "F.Cu") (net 6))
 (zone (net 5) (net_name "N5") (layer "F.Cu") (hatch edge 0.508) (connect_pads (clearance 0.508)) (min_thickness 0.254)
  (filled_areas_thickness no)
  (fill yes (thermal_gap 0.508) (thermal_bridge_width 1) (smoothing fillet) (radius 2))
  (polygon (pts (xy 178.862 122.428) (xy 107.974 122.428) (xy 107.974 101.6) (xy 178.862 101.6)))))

